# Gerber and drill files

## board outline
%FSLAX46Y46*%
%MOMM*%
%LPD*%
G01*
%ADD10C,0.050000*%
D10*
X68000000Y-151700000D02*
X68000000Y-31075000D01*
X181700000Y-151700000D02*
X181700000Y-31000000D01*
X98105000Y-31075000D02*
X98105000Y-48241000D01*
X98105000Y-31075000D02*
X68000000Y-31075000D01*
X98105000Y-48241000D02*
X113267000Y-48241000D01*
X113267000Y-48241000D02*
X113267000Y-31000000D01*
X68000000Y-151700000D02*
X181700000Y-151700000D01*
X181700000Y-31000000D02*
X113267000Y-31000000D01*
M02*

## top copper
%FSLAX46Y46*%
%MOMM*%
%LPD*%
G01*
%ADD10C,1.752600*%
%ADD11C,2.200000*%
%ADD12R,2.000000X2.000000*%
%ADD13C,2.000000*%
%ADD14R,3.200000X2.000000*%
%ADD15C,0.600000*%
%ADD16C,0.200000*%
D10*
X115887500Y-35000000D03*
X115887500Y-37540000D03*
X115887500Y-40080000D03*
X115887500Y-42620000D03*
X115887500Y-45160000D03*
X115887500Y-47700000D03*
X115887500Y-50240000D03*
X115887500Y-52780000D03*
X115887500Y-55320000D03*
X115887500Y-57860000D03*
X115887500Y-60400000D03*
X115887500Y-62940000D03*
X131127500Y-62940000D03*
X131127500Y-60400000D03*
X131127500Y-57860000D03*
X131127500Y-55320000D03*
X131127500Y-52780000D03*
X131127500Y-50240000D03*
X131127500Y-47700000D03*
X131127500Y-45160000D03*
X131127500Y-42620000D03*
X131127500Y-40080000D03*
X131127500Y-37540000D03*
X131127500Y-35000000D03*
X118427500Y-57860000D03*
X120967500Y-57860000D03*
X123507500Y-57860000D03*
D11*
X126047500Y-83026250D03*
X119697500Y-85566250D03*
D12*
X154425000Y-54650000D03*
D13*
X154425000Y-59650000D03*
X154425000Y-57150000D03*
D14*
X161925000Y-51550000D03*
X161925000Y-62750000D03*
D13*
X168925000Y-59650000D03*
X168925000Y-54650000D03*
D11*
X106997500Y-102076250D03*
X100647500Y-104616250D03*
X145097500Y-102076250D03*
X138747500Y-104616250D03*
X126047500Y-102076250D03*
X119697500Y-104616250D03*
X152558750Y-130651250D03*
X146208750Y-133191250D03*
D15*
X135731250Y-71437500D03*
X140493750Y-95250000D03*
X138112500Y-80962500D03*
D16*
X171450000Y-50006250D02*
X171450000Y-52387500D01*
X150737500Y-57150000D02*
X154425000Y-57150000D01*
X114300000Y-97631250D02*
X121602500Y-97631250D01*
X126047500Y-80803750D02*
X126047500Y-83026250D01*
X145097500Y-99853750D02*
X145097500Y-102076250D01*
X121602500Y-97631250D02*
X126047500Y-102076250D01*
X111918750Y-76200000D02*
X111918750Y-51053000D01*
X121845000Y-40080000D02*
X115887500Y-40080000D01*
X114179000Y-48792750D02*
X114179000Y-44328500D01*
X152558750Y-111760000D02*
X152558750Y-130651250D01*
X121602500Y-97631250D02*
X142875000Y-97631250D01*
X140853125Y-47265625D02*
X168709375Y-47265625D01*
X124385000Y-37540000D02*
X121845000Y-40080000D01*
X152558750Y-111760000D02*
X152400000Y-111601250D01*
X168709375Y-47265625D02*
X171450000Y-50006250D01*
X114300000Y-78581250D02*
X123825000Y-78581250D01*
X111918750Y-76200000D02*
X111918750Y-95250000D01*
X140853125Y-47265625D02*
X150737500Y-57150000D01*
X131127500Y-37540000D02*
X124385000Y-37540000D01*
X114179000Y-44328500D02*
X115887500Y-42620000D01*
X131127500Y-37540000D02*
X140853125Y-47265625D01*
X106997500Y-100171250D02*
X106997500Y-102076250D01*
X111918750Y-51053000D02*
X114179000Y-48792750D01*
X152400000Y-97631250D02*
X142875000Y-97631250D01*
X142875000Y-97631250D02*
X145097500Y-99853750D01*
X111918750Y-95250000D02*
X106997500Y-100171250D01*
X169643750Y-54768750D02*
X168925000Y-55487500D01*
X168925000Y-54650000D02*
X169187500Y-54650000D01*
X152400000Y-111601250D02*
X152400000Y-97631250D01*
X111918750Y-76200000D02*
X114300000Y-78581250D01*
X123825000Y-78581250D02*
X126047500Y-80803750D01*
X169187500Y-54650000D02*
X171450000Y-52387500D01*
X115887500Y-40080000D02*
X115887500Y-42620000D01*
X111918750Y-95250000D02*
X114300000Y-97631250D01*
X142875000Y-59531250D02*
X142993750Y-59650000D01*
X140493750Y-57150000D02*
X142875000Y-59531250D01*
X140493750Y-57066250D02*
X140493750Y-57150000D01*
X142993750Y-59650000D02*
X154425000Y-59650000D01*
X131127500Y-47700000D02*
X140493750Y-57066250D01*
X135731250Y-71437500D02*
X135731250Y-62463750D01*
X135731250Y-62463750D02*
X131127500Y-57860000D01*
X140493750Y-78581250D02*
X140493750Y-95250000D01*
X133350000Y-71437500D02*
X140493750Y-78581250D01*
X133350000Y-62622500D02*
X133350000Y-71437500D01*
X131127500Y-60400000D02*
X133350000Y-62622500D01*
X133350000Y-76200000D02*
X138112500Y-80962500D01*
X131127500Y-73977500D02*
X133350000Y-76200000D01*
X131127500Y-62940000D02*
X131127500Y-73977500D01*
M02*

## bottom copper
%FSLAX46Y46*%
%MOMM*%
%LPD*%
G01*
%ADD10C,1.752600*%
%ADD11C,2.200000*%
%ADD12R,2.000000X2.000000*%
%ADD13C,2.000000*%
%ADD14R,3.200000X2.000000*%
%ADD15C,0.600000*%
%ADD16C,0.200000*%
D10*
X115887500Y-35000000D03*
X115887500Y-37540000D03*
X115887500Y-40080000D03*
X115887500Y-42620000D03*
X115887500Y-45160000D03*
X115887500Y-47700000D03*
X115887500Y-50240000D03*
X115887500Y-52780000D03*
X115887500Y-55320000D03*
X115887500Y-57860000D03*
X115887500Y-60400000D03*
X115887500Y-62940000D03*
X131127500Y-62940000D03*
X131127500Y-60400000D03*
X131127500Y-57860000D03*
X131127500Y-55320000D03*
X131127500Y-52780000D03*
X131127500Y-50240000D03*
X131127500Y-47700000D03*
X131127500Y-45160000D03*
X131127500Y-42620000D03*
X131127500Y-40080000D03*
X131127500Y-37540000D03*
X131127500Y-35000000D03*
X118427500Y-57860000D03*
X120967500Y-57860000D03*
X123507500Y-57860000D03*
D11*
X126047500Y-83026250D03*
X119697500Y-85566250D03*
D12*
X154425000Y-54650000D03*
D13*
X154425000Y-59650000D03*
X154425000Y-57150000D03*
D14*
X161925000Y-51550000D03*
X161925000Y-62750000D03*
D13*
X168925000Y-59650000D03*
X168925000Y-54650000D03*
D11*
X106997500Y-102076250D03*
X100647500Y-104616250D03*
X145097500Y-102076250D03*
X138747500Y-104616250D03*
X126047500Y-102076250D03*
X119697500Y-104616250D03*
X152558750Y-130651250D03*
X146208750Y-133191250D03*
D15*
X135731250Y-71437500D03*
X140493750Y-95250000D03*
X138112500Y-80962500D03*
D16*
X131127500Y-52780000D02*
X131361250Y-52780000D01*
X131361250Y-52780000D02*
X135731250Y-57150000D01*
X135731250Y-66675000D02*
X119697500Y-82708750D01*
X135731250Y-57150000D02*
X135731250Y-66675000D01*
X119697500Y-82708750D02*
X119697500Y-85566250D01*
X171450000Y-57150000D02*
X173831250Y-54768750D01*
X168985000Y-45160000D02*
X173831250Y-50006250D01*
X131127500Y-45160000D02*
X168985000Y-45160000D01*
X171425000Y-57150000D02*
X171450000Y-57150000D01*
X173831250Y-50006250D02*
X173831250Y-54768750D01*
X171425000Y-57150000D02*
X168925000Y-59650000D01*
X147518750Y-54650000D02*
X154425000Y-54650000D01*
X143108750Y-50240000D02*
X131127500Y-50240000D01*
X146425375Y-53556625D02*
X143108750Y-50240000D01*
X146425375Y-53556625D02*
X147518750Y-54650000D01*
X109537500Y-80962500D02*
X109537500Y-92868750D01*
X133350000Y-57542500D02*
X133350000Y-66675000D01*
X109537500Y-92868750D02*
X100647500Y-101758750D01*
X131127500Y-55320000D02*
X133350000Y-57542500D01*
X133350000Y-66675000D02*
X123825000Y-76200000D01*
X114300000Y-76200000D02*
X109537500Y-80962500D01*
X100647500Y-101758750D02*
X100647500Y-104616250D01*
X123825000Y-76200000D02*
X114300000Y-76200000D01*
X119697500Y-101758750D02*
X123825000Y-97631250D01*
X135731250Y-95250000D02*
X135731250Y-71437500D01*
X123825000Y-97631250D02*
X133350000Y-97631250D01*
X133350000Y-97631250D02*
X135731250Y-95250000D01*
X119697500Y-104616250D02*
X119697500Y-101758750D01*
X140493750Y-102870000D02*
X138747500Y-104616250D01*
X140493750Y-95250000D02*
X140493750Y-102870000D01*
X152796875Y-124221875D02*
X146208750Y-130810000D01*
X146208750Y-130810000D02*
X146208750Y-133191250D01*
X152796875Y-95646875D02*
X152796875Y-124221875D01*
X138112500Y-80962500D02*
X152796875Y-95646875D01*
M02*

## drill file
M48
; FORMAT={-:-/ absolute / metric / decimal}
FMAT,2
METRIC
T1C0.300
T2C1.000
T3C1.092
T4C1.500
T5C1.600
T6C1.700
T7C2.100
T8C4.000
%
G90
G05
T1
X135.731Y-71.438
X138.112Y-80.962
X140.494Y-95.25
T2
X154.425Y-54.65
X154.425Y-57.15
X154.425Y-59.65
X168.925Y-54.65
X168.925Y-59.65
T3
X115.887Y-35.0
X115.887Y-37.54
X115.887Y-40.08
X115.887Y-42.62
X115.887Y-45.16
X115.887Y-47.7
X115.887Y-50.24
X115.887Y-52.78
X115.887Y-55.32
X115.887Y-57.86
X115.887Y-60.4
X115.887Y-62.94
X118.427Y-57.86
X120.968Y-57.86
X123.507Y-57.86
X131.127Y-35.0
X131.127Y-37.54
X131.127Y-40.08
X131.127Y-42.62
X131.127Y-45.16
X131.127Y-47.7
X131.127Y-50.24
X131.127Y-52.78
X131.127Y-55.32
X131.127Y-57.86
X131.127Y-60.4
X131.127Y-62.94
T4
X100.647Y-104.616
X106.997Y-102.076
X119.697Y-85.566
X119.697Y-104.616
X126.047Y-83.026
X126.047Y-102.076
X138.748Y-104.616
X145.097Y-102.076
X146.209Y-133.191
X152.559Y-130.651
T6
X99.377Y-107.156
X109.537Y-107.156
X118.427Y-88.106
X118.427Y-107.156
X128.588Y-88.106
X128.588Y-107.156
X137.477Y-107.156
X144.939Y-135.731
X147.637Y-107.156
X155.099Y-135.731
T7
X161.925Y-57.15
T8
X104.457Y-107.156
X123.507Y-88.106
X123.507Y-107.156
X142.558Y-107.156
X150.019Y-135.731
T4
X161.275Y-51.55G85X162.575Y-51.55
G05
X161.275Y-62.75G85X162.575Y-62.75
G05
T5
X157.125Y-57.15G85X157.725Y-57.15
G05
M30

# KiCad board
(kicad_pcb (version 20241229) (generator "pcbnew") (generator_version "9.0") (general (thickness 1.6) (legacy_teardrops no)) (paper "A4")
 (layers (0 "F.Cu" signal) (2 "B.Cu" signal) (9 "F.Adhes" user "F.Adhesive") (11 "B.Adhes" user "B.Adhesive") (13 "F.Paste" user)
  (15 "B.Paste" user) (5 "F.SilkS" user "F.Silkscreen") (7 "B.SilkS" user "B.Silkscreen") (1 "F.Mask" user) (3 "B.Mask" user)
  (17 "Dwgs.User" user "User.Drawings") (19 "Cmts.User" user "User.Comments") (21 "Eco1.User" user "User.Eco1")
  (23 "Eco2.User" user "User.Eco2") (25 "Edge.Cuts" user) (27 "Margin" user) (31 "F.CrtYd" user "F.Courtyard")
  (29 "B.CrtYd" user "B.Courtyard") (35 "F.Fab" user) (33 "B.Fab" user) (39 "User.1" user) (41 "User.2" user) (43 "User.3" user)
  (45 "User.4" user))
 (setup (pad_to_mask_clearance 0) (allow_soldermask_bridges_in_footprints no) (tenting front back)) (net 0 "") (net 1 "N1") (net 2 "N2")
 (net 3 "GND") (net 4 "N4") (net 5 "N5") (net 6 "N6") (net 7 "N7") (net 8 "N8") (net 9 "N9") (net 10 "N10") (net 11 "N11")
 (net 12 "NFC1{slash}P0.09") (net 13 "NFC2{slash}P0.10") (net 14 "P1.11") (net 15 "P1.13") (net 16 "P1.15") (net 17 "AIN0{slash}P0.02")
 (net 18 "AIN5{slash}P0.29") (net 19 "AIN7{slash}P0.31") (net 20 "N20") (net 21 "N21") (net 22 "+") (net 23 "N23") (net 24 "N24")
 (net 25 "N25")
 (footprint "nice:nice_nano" (layer "F.Cu") (at 123.5075 48.97 -90)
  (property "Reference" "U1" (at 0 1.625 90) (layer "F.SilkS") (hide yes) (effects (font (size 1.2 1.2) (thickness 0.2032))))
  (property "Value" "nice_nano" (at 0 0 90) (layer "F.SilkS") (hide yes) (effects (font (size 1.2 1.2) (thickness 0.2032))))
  (pad "1" thru_hole circle (at -13.97 7.62 270) (size 1.7526 1.7526) (drill 1.0922) (layers "*.Cu" "*.SilkS" "*.Mask")
   (remove_unused_layers no) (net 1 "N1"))
  (pad "2" thru_hole circle (at -11.43 7.62 270) (size 1.7526 1.7526) (drill 1.0922) (layers "*.Cu" "*.SilkS" "*.Mask")
   (remove_unused_layers no) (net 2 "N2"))
  (pad "3" thru_hole circle (at -8.89 7.62 270) (size 1.7526 1.7526) (drill 1.0922) (layers "*.Cu" "*.SilkS" "*.Mask")
   (remove_unused_layers no) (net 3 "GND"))
  (pad "4" thru_hole circle (at -6.35 7.62 270) (size 1.7526 1.7526) (drill 1.0922) (layers "*.Cu" "*.SilkS" "*.Mask")
   (remove_unused_layers no) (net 3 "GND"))
  (pad "5" thru_hole circle (at -3.81 7.62 270) (size 1.7526 1.7526) (drill 1.0922) (layers "*.Cu" "*.SilkS" "*.Mask")
   (remove_unused_layers no) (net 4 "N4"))
  (pad "6" thru_hole circle (at -1.27 7.62 270) (size 1.7526 1.7526) (drill 1.0922) (layers "*.Cu" "*.SilkS" "*.Mask")
   (remove_unused_layers no) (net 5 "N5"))
  (pad "7" thru_hole circle (at 1.27 7.62 270) (size 1.7526 1.7526) (drill 1.0922) (layers "*.Cu" "*.SilkS" "*.Mask")
   (remove_unused_layers no) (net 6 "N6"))
  (pad "8" thru_hole circle (at 3.81 7.62 270) (size 1.7526 1.7526) (drill 1.0922) (layers "*.Cu" "*.SilkS" "*.Mask")
   (remove_unused_layers no) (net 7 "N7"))
  (pad "9" thru_hole circle (at 6.35 7.62 270) (size 1.7526 1.7526) (drill 1.0922) (layers "*.Cu" "*.SilkS" "*.Mask")
   (remove_unused_layers no) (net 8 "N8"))
  (pad "10" thru_hole circle (at 8.89 7.62 270) (size 1.7526 1.7526) (drill 1.0922) (layers "*.Cu" "*.SilkS" "*.Mask")
   (remove_unused_layers no) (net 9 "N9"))
  (pad "11" thru_hole circle (at 11.43 7.62 270) (size 1.7526 1.7526) (drill 1.0922) (layers "*.Cu" "*.SilkS" "*.Mask")
   (remove_unused_layers no) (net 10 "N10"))
  (pad "12" thru_hole circle (at 13.97 7.62 270) (size 1.7526 1.7526) (drill 1.0922) (layers "*.Cu" "*.SilkS" "*.Mask")
   (remove_unused_layers no) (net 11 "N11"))
  (pad "13" thru_hole circle (at 13.97 -7.62 270) (size 1.7526 1.7526) (drill 1.0922) (layers "*.Cu" "*.SilkS" "*.Mask")
   (remove_unused_layers no) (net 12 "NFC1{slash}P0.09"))
  (pad "14" thru_hole circle (at 11.43 -7.62 270) (size 1.7526 1.7526) (drill 1.0922) (layers "*.Cu" "*.SilkS" "*.Mask")
   (remove_unused_layers no) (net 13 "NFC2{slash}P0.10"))
  (pad "15" thru_hole circle (at 8.89 -7.62 270) (size 1.7526 1.7526) (drill 1.0922) (layers "*.Cu" "*.SilkS" "*.Mask")
   (remove_unused_layers no) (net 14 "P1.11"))
  (pad "16" thru_hole circle (at 6.35 -7.62 270) (size 1.7526 1.7526) (drill 1.0922) (layers "*.Cu" "*.SilkS" "*.Mask")
   (remove_unused_layers no) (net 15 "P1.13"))
  (pad "17" thru_hole circle (at 3.81 -7.62 270) (size 1.7526 1.7526) (drill 1.0922) (layers "*.Cu" "*.SilkS" "*.Mask")
   (remove_unused_layers no) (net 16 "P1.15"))
  (pad "18" thru_hole circle (at 1.27 -7.62 270) (size 1.7526 1.7526) (drill 1.0922) (layers "*.Cu" "*.SilkS" "*.Mask")
   (remove_unused_layers no) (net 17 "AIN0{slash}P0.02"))
  (pad "19" thru_hole circle (at -1.27 -7.62 270) (size 1.7526 1.7526) (drill 1.0922) (layers "*.Cu" "*.SilkS" "*.Mask")
   (remove_unused_layers no) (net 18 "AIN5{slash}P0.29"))
  (pad "20" thru_hole circle (at -3.81 -7.62 270) (size 1.7526 1.7526) (drill 1.0922) (layers "*.Cu" "*.SilkS" "*.Mask")
   (remove_unused_layers no) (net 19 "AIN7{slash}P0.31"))
  (pad "21" thru_hole circle (at -6.35 -7.62 270) (size 1.7526 1.7526) (drill 1.0922) (layers "*.Cu" "*.SilkS" "*.Mask")
   (remove_unused_layers no) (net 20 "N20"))
  (pad "22" thru_hole circle (at -8.89 -7.62 270) (size 1.7526 1.7526) (drill 1.0922) (layers "*.Cu" "*.SilkS" "*.Mask")
   (remove_unused_layers no) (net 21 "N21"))
  (pad "23" thru_hole circle (at -11.43 -7.62 270) (size 1.7526 1.7526) (drill 1.0922) (layers "*.Cu" "*.SilkS" "*.Mask")
   (remove_unused_layers no) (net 3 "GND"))
  (pad "24" thru_hole circle (at -13.97 -7.62 270) (size 1.7526 1.7526) (drill 1.0922) (layers "*.Cu" "*.SilkS" "*.Mask")
   (remove_unused_layers no) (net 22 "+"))
  (pad "31" thru_hole circle (at 8.89 5.08 270) (size 1.7526 1.7526) (drill 1.0922) (layers "*.Cu" "*.SilkS" "*.Mask")
   (remove_unused_layers no) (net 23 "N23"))
  (pad "32" thru_hole circle (at 8.89 2.54 270) (size 1.7526 1.7526) (drill 1.0922) (layers "*.Cu" "*.SilkS" "*.Mask")
   (remove_unused_layers no) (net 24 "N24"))
  (pad "33" thru_hole circle (at 8.89 0 270) (size 1.7526 1.7526) (drill 1.0922) (layers "*.Cu" "*.SilkS" "*.Mask")
   (remove_unused_layers no) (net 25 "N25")))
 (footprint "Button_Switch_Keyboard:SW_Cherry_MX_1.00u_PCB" (layer "F.Cu") (at 126.0475 83.02625)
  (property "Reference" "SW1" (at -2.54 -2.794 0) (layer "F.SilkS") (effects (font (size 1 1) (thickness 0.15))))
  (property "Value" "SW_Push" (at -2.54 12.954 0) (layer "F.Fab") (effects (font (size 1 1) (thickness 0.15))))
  (pad "" np_thru_hole circle (at -7.62 5.08) (size 1.7 1.7) (drill 1.7) (layers "*.Cu" "*.Mask"))
  (pad "" np_thru_hole circle (at -2.54 5.08) (size 4 4) (drill 4) (layers "*.Cu" "*.Mask"))
  (pad "" np_thru_hole circle (at 2.54 5.08) (size 1.7 1.7) (drill 1.7) (layers "*.Cu" "*.Mask"))
  (pad "1" thru_hole circle (at 0 0) (size 2.2 2.2) (drill 1.5) (layers "*.Cu" "*.Mask") (remove_unused_layers no) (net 3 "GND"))
  (pad "2" thru_hole circle (at -6.35 2.54) (size 2.2 2.2) (drill 1.5) (layers "*.Cu" "*.Mask") (remove_unused_layers no) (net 16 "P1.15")))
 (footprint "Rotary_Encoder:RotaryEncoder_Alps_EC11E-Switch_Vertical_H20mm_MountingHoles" (layer "F.Cu") (at 154.425 54.65)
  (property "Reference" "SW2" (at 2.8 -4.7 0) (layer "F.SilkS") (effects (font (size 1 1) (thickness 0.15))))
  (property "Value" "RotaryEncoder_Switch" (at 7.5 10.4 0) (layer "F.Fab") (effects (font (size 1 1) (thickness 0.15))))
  (pad "" np_thru_hole oval (at 3 2.5) (size 2.2 1.6) (drill oval 2.2 1.6) (layers "*.Mask"))
  (pad "" np_thru_hole circle (at 7.5 2.5) (size 2.1 2.1) (drill 2.1) (layers "*.Mask"))
  (pad "A" thru_hole rect (at 0 0) (size 2 2) (drill 1) (layers "*.Cu" "*.Mask") (remove_unused_layers no) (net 17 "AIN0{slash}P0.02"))
  (pad "B" thru_hole circle (at 0 5) (size 2 2) (drill 1) (layers "*.Cu" "*.Mask") (remove_unused_layers no) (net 18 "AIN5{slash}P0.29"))
  (pad "C" thru_hole circle (at 0 2.5) (size 2 2) (drill 1) (layers "*.Cu" "*.Mask") (remove_unused_layers no) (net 3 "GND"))
  (pad "MP" thru_hole rect (at 7.5 -3.1) (size 3.2 2) (drill oval 2.8 1.5) (layers "*.Cu" "*.Mask") (remove_unused_layers no))
  (pad "MP" thru_hole rect (at 7.5 8.1) (size 3.2 2) (drill oval 2.8 1.5) (layers "*.Cu" "*.Mask") (remove_unused_layers no))
  (pad "S1" thru_hole circle (at 14.5 5) (size 2 2) (drill 1) (layers "*.Cu" "*.Mask") (remove_unused_layers no) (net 19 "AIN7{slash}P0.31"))
  (pad "S2" thru_hole circle (at 14.5 0) (size 2 2) (drill 1) (layers "*.Cu" "*.Mask") (remove_unused_layers no) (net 3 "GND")))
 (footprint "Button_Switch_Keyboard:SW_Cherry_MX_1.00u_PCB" (layer "F.Cu") (at 106.9975 102.07625)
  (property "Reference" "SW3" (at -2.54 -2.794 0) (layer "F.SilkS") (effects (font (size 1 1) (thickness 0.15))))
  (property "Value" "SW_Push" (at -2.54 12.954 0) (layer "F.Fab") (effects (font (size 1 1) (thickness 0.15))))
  (pad "" np_thru_hole circle (at -7.62 5.08) (size 1.7 1.7) (drill 1.7) (layers "*.Cu" "*.Mask"))
  (pad "" np_thru_hole circle (at -2.54 5.08) (size 4 4) (drill 4) (layers "*.Cu" "*.Mask"))
  (pad "" np_thru_hole circle (at 2.54 5.08) (size 1.7 1.7) (drill 1.7) (layers "*.Cu" "*.Mask"))
  (pad "1" thru_hole circle (at 0 0) (size 2.2 2.2) (drill 1.5) (layers "*.Cu" "*.Mask") (remove_unused_layers no) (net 3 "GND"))
  (pad "2" thru_hole circle (at -6.35 2.54) (size 2.2 2.2) (drill 1.5) (layers "*.Cu" "*.Mask") (remove_unused_layers no) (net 15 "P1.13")))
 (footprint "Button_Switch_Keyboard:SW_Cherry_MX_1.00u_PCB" (layer "F.Cu") (at 145.0975 102.07625)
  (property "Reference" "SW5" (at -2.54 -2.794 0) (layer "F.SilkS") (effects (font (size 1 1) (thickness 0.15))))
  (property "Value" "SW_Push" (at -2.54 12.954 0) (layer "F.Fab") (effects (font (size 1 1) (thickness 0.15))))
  (pad "" np_thru_hole circle (at -7.62 5.08) (size 1.7 1.7) (drill 1.7) (layers "*.Cu" "*.Mask"))
  (pad "" np_thru_hole circle (at -2.54 5.08) (size 4 4) (drill 4) (layers "*.Cu" "*.Mask"))
  (pad "" np_thru_hole circle (at 2.54 5.08) (size 1.7 1.7) (drill 1.7) (layers "*.Cu" "*.Mask"))
  (pad "1" thru_hole circle (at 0 0) (size 2.2 2.2) (drill 1.5) (layers "*.Cu" "*.Mask") (remove_unused_layers no) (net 3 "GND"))
  (pad "2" thru_hole circle (at -6.35 2.54) (size 2.2 2.2) (drill 1.5) (layers "*.Cu" "*.Mask") (remove_unused_layers no)
   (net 13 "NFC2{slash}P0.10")))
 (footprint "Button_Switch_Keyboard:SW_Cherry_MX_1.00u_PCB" (layer "F.Cu") (at 126.0475 102.07625)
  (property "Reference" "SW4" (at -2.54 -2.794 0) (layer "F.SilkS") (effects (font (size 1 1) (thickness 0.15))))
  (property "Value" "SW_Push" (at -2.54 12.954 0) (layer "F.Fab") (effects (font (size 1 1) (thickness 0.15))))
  (pad "" np_thru_hole circle (at -7.62 5.08) (size 1.7 1.7) (drill 1.7) (layers "*.Cu" "*.Mask"))
  (pad "" np_thru_hole circle (at -2.54 5.08) (size 4 4) (drill 4) (layers "*.Cu" "*.Mask"))
  (pad "" np_thru_hole circle (at 2.54 5.08) (size 1.7 1.7) (drill 1.7) (layers "*.Cu" "*.Mask"))
  (pad "1" thru_hole circle (at 0 0) (size 2.2 2.2) (drill 1.5) (layers "*.Cu" "*.Mask") (remove_unused_layers no) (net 3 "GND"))
  (pad "2" thru_hole circle (at -6.35 2.54) (size 2.2 2.2) (drill 1.5) (layers "*.Cu" "*.Mask") (remove_unused_layers no) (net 14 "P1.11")))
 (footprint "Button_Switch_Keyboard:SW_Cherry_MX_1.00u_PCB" (layer "F.Cu") (at 152.55875 130.65125)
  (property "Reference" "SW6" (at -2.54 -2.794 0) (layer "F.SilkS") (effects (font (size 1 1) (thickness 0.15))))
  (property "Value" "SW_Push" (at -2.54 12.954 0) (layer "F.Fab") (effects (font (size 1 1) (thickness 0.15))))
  (pad "" np_thru_hole circle (at -7.62 5.08) (size 1.7 1.7) (drill 1.7) (layers "*.Cu" "*.Mask"))
  (pad "" np_thru_hole circle (at -2.54 5.08) (size 4 4) (drill 4) (layers "*.Cu" "*.Mask"))
  (pad "" np_thru_hole circle (at 2.54 5.08) (size 1.7 1.7) (drill 1.7) (layers "*.Cu" "*.Mask"))
  (pad "1" thru_hole circle (at 0 0) (size 2.2 2.2) (drill 1.5) (layers "*.Cu" "*.Mask") (remove_unused_layers no) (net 3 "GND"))
  (pad "2" thru_hole circle (at -6.35 2.54) (size 2.2 2.2) (drill 1.5) (layers "*.Cu" "*.Mask") (remove_unused_layers no)
   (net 12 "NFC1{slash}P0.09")))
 (gr_line (start 68 151.7) (end 68 31.075) (stroke (width 0.05) (type default)) (layer "Edge.Cuts"))
 (gr_line (start 181.7 151.7) (end 181.7 31) (stroke (width 0.05) (type default)) (layer "Edge.Cuts"))
 (gr_line (start 98.105 31.075) (end 98.105 48.241) (stroke (width 0.05) (type default)) (layer "Edge.Cuts"))
 (gr_line (start 98.105 31.075) (end 68 31.075) (stroke (width 0.05) (type default)) (layer "Edge.Cuts"))
 (gr_line (start 98.105 48.241) (end 113.267 48.241) (stroke (width 0.05) (type default)) (layer "Edge.Cuts"))
 (gr_line (start 113.267 48.241) (end 113.267 31) (stroke (width 0.05) (type default)) (layer "Edge.Cuts"))
 (gr_line (start 68 151.7) (end 181.7 151.7) (stroke (width 0.05) (type default)) (layer "Edge.Cuts"))
 (gr_line (start 181.7 31) (end 113.267 31) (stroke (width 0.05) (type default)) (layer "Edge.Cuts"))
 (segment (start 131.1275 52.78) (end 131.36125 52.78) (width 0.2) (layer "B.Cu") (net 16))
 (segment (start 131.36125 52.78) (end 135.73125 57.15) (width 0.2) (layer "B.Cu") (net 16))
 (segment (start 135.73125 66.675) (end 119.6975 82.70875) (width 0.2) (layer "B.Cu") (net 16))
 (segment (start 135.73125 57.15) (end 135.73125 66.675) (width 0.2) (layer "B.Cu") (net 16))
 (segment (start 119.6975 82.70875) (end 119.6975 85.56625) (width 0.2) (layer "B.Cu") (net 16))
 (segment (start 171.45 50.00625) (end 171.45 52.3875) (width 0.2) (layer "F.Cu") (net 3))
 (segment (start 150.7375 57.15) (end 154.425 57.15) (width 0.2) (layer "F.Cu") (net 3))
 (segment (start 114.3 97.63125) (end 121.6025 97.63125) (width 0.2) (layer "F.Cu") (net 3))
 (segment (start 126.0475 80.80375) (end 126.0475 83.02625) (width 0.2) (layer "F.Cu") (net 3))
 (segment (start 145.0975 99.85375) (end 145.0975 102.07625) (width 0.2) (layer "F.Cu") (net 3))
 (segment (start 121.6025 97.63125) (end 126.0475 102.07625) (width 0.2) (layer "F.Cu") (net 3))
 (segment (start 111.91875 76.2) (end 111.91875 51.053) (width 0.2) (layer "F.Cu") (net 3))
 (segment (start 121.845 40.08) (end 115.8875 40.08) (width 0.2) (layer "F.Cu") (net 3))
 (segment (start 114.179 48.79275) (end 114.179 44.3285) (width 0.2) (layer "F.Cu") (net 3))
 (segment (start 152.55875 111.76) (end 152.55875 130.65125) (width 0.2) (layer "F.Cu") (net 3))
 (segment (start 121.6025 97.63125) (end 142.875 97.63125) (width 0.2) (layer "F.Cu") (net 3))
 (segment (start 140.853125 47.265625) (end 168.709375 47.265625) (width 0.2) (layer "F.Cu") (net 3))
 (segment (start 124.385 37.54) (end 121.845 40.08) (width 0.2) (layer "F.Cu") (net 3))
 (segment (start 152.55875 111.76) (end 152.4 111.60125) (width 0.2) (layer "F.Cu") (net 3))
 (segment (start 168.709375 47.265625) (end 171.45 50.00625) (width 0.2) (layer "F.Cu") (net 3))
 (segment (start 114.3 78.58125) (end 123.825 78.58125) (width 0.2) (layer "F.Cu") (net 3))
 (segment (start 111.91875 76.2) (end 111.91875 95.25) (width 0.2) (layer "F.Cu") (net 3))
 (segment (start 140.853125 47.265625) (end 150.7375 57.15) (width 0.2) (layer "F.Cu") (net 3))
 (segment (start 131.1275 37.54) (end 124.385 37.54) (width 0.2) (layer "F.Cu") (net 3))
 (segment (start 114.179 44.3285) (end 115.8875 42.62) (width 0.2) (layer "F.Cu") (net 3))
 (segment (start 131.1275 37.54) (end 140.853125 47.265625) (width 0.2) (layer "F.Cu") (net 3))
 (segment (start 106.9975 100.17125) (end 106.9975 102.07625) (width 0.2) (layer "F.Cu") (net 3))
 (segment (start 111.91875 51.053) (end 114.179 48.79275) (width 0.2) (layer "F.Cu") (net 3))
 (segment (start 152.4 97.63125) (end 142.875 97.63125) (width 0.2) (layer "F.Cu") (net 3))
 (segment (start 142.875 97.63125) (end 145.0975 99.85375) (width 0.2) (layer "F.Cu") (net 3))
 (segment (start 111.91875 95.25) (end 106.9975 100.17125) (width 0.2) (layer "F.Cu") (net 3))
 (segment (start 169.64375 54.76875) (end 168.925 55.4875) (width 0.2) (layer "F.Cu") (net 3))
 (segment (start 168.925 54.65) (end 169.1875 54.65) (width 0.2) (layer "F.Cu") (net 3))
 (segment (start 152.4 111.60125) (end 152.4 97.63125) (width 0.2) (layer "F.Cu") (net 3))
 (segment (start 111.91875 76.2) (end 114.3 78.58125) (width 0.2) (layer "F.Cu") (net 3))
 (segment (start 123.825 78.58125) (end 126.0475 80.80375) (width 0.2) (layer "F.Cu") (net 3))
 (segment (start 169.1875 54.65) (end 171.45 52.3875) (width 0.2) (layer "F.Cu") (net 3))
 (segment (start 115.8875 40.08) (end 115.8875 42.62) (width 0.2) (layer "F.Cu") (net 3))
 (segment (start 111.91875 95.25) (end 114.3 97.63125) (width 0.2) (layer "F.Cu") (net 3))
 (segment (start 142.875 59.53125) (end 142.99375 59.65) (width 0.2) (layer "F.Cu") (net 18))
 (segment (start 140.49375 57.15) (end 142.875 59.53125) (width 0.2) (layer "F.Cu") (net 18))
 (segment (start 140.49375 57.06625) (end 140.49375 57.15) (width 0.2) (layer "F.Cu") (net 18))
 (segment (start 142.99375 59.65) (end 154.425 59.65) (width 0.2) (layer "F.Cu") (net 18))
 (segment (start 131.1275 47.7) (end 140.49375 57.06625) (width 0.2) (layer "F.Cu") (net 18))
 (segment (start 171.45 57.15) (end 173.83125 54.76875) (width 0.2) (layer "B.Cu") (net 19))
 (segment (start 168.985 45.16) (end 173.83125 50.00625) (width 0.2) (layer "B.Cu") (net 19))
 (segment (start 131.1275 45.16) (end 168.985 45.16) (width 0.2) (layer "B.Cu") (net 19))
 (segment (start 171.425 57.15) (end 171.45 57.15) (width 0.2) (layer "B.Cu") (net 19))
 (segment (start 173.83125 50.00625) (end 173.83125 54.76875) (width 0.2) (layer "B.Cu") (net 19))
 (segment (start 171.425 57.15) (end 168.925 59.65) (width 0.2) (layer "B.Cu") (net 19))
 (segment (start 147.51875 54.65) (end 154.425 54.65) (width 0.2) (layer "B.Cu") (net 17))
 (segment (start 143.10875 50.24) (end 131.1275 50.24) (width 0.2) (layer "B.Cu") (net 17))
 (segment (start 146.425375 53.556625) (end 143.10875 50.24) (width 0.2) (layer "B.Cu") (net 17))
 (segment (start 146.425375 53.556625) (end 147.51875 54.65) (width 0.2) (layer "B.Cu") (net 17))
 (segment (start 109.5375 80.9625) (end 109.5375 92.86875) (width 0.2) (layer "B.Cu") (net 15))
 (segment (start 133.35 57.5425) (end 133.35 66.675) (width 0.2) (layer "B.Cu") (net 15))
 (segment (start 109.5375 92.86875) (end 100.6475 101.75875) (width 0.2) (layer "B.Cu") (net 15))
 (segment (start 131.1275 55.32) (end 133.35 57.5425) (width 0.2) (layer "B.Cu") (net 15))
 (segment (start 133.35 66.675) (end 123.825 76.2) (width 0.2) (layer "B.Cu") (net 15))
 (segment (start 114.3 76.2) (end 109.5375 80.9625) (width 0.2) (layer "B.Cu") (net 15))
 (segment (start 100.6475 101.75875) (end 100.6475 104.61625) (width 0.2) (layer "B.Cu") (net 15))
 (segment (start 123.825 76.2) (end 114.3 76.2) (width 0.2) (layer "B.Cu") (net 15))
 (segment (start 135.73125 71.4375) (end 135.73125 62.46375) (width 0.2) (layer "F.Cu") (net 14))
 (segment (start 135.73125 62.46375) (end 131.1275 57.86) (width 0.2) (layer "F.Cu") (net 14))
 (via (at 135.73125 71.4375) (size 0.6) (drill 0.3) (layers "F.Cu" "B.Cu") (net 14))
 (segment (start 119.6975 101.75875) (end 123.825 97.63125) (width 0.2) (layer "B.Cu") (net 14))
 (segment (start 135.73125 95.25) (end 135.73125 71.4375) (width 0.2) (layer "B.Cu") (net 14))
 (segment (start 123.825 97.63125) (end 133.35 97.63125) (width 0.2) (layer "B.Cu") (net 14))
 (segment (start 133.35 97.63125) (end 135.73125 95.25) (width 0.2) (layer "B.Cu") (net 14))
 (segment (start 119.6975 104.61625) (end 119.6975 101.75875) (width 0.2) (layer "B.Cu") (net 14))
 (segment (start 140.49375 78.58125) (end 140.49375 95.25) (width 0.2) (layer "F.Cu") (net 13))
 (segment (start 133.35 71.4375) (end 140.49375 78.58125) (width 0.2) (layer "F.Cu") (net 13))
 (segment (start 133.35 62.6225) (end 133.35 71.4375) (width 0.2) (layer "F.Cu") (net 13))
 (segment (start 131.1275 60.4) (end 133.35 62.6225) (width 0.2) (layer "F.Cu") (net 13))
 (via (at 140.49375 95.25) (size 0.6) (drill 0.3) (layers "F.Cu" "B.Cu") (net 13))
 (segment (start 140.49375 102.87) (end 138.7475 104.61625) (width 0.2) (layer "B.Cu") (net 13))
 (segment (start 140.49375 95.25) (end 140.49375 102.87) (width 0.2) (layer "B.Cu") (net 13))
 (segment (start 133.35 76.2) (end 138.1125 80.9625) (width 0.2) (layer "F.Cu") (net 12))
 (segment (start 131.1275 73.9775) (end 133.35 76.2) (width 0.2) (layer "F.Cu") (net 12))
 (segment (start 131.1275 62.94) (end 131.1275 73.9775) (width 0.2) (layer "F.Cu") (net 12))
 (via (at 138.1125 80.9625) (size 0.6) (drill 0.3) (layers "F.Cu" "B.Cu") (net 12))
 (segment (start 152.796875 124.221875) (end 146.20875 130.81) (width 0.2) (layer "B.Cu") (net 12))
 (segment (start 146.20875 130.81) (end 146.20875 133.19125) (width 0.2) (layer "B.Cu") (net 12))
 (segment (start 152.796875 95.646875) (end 152.796875 124.221875) (width 0.2) (layer "B.Cu") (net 12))
 (segment (start 138.1125 80.9625) (end 152.796875 95.646875) (width 0.2) (layer "B.Cu") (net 12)))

